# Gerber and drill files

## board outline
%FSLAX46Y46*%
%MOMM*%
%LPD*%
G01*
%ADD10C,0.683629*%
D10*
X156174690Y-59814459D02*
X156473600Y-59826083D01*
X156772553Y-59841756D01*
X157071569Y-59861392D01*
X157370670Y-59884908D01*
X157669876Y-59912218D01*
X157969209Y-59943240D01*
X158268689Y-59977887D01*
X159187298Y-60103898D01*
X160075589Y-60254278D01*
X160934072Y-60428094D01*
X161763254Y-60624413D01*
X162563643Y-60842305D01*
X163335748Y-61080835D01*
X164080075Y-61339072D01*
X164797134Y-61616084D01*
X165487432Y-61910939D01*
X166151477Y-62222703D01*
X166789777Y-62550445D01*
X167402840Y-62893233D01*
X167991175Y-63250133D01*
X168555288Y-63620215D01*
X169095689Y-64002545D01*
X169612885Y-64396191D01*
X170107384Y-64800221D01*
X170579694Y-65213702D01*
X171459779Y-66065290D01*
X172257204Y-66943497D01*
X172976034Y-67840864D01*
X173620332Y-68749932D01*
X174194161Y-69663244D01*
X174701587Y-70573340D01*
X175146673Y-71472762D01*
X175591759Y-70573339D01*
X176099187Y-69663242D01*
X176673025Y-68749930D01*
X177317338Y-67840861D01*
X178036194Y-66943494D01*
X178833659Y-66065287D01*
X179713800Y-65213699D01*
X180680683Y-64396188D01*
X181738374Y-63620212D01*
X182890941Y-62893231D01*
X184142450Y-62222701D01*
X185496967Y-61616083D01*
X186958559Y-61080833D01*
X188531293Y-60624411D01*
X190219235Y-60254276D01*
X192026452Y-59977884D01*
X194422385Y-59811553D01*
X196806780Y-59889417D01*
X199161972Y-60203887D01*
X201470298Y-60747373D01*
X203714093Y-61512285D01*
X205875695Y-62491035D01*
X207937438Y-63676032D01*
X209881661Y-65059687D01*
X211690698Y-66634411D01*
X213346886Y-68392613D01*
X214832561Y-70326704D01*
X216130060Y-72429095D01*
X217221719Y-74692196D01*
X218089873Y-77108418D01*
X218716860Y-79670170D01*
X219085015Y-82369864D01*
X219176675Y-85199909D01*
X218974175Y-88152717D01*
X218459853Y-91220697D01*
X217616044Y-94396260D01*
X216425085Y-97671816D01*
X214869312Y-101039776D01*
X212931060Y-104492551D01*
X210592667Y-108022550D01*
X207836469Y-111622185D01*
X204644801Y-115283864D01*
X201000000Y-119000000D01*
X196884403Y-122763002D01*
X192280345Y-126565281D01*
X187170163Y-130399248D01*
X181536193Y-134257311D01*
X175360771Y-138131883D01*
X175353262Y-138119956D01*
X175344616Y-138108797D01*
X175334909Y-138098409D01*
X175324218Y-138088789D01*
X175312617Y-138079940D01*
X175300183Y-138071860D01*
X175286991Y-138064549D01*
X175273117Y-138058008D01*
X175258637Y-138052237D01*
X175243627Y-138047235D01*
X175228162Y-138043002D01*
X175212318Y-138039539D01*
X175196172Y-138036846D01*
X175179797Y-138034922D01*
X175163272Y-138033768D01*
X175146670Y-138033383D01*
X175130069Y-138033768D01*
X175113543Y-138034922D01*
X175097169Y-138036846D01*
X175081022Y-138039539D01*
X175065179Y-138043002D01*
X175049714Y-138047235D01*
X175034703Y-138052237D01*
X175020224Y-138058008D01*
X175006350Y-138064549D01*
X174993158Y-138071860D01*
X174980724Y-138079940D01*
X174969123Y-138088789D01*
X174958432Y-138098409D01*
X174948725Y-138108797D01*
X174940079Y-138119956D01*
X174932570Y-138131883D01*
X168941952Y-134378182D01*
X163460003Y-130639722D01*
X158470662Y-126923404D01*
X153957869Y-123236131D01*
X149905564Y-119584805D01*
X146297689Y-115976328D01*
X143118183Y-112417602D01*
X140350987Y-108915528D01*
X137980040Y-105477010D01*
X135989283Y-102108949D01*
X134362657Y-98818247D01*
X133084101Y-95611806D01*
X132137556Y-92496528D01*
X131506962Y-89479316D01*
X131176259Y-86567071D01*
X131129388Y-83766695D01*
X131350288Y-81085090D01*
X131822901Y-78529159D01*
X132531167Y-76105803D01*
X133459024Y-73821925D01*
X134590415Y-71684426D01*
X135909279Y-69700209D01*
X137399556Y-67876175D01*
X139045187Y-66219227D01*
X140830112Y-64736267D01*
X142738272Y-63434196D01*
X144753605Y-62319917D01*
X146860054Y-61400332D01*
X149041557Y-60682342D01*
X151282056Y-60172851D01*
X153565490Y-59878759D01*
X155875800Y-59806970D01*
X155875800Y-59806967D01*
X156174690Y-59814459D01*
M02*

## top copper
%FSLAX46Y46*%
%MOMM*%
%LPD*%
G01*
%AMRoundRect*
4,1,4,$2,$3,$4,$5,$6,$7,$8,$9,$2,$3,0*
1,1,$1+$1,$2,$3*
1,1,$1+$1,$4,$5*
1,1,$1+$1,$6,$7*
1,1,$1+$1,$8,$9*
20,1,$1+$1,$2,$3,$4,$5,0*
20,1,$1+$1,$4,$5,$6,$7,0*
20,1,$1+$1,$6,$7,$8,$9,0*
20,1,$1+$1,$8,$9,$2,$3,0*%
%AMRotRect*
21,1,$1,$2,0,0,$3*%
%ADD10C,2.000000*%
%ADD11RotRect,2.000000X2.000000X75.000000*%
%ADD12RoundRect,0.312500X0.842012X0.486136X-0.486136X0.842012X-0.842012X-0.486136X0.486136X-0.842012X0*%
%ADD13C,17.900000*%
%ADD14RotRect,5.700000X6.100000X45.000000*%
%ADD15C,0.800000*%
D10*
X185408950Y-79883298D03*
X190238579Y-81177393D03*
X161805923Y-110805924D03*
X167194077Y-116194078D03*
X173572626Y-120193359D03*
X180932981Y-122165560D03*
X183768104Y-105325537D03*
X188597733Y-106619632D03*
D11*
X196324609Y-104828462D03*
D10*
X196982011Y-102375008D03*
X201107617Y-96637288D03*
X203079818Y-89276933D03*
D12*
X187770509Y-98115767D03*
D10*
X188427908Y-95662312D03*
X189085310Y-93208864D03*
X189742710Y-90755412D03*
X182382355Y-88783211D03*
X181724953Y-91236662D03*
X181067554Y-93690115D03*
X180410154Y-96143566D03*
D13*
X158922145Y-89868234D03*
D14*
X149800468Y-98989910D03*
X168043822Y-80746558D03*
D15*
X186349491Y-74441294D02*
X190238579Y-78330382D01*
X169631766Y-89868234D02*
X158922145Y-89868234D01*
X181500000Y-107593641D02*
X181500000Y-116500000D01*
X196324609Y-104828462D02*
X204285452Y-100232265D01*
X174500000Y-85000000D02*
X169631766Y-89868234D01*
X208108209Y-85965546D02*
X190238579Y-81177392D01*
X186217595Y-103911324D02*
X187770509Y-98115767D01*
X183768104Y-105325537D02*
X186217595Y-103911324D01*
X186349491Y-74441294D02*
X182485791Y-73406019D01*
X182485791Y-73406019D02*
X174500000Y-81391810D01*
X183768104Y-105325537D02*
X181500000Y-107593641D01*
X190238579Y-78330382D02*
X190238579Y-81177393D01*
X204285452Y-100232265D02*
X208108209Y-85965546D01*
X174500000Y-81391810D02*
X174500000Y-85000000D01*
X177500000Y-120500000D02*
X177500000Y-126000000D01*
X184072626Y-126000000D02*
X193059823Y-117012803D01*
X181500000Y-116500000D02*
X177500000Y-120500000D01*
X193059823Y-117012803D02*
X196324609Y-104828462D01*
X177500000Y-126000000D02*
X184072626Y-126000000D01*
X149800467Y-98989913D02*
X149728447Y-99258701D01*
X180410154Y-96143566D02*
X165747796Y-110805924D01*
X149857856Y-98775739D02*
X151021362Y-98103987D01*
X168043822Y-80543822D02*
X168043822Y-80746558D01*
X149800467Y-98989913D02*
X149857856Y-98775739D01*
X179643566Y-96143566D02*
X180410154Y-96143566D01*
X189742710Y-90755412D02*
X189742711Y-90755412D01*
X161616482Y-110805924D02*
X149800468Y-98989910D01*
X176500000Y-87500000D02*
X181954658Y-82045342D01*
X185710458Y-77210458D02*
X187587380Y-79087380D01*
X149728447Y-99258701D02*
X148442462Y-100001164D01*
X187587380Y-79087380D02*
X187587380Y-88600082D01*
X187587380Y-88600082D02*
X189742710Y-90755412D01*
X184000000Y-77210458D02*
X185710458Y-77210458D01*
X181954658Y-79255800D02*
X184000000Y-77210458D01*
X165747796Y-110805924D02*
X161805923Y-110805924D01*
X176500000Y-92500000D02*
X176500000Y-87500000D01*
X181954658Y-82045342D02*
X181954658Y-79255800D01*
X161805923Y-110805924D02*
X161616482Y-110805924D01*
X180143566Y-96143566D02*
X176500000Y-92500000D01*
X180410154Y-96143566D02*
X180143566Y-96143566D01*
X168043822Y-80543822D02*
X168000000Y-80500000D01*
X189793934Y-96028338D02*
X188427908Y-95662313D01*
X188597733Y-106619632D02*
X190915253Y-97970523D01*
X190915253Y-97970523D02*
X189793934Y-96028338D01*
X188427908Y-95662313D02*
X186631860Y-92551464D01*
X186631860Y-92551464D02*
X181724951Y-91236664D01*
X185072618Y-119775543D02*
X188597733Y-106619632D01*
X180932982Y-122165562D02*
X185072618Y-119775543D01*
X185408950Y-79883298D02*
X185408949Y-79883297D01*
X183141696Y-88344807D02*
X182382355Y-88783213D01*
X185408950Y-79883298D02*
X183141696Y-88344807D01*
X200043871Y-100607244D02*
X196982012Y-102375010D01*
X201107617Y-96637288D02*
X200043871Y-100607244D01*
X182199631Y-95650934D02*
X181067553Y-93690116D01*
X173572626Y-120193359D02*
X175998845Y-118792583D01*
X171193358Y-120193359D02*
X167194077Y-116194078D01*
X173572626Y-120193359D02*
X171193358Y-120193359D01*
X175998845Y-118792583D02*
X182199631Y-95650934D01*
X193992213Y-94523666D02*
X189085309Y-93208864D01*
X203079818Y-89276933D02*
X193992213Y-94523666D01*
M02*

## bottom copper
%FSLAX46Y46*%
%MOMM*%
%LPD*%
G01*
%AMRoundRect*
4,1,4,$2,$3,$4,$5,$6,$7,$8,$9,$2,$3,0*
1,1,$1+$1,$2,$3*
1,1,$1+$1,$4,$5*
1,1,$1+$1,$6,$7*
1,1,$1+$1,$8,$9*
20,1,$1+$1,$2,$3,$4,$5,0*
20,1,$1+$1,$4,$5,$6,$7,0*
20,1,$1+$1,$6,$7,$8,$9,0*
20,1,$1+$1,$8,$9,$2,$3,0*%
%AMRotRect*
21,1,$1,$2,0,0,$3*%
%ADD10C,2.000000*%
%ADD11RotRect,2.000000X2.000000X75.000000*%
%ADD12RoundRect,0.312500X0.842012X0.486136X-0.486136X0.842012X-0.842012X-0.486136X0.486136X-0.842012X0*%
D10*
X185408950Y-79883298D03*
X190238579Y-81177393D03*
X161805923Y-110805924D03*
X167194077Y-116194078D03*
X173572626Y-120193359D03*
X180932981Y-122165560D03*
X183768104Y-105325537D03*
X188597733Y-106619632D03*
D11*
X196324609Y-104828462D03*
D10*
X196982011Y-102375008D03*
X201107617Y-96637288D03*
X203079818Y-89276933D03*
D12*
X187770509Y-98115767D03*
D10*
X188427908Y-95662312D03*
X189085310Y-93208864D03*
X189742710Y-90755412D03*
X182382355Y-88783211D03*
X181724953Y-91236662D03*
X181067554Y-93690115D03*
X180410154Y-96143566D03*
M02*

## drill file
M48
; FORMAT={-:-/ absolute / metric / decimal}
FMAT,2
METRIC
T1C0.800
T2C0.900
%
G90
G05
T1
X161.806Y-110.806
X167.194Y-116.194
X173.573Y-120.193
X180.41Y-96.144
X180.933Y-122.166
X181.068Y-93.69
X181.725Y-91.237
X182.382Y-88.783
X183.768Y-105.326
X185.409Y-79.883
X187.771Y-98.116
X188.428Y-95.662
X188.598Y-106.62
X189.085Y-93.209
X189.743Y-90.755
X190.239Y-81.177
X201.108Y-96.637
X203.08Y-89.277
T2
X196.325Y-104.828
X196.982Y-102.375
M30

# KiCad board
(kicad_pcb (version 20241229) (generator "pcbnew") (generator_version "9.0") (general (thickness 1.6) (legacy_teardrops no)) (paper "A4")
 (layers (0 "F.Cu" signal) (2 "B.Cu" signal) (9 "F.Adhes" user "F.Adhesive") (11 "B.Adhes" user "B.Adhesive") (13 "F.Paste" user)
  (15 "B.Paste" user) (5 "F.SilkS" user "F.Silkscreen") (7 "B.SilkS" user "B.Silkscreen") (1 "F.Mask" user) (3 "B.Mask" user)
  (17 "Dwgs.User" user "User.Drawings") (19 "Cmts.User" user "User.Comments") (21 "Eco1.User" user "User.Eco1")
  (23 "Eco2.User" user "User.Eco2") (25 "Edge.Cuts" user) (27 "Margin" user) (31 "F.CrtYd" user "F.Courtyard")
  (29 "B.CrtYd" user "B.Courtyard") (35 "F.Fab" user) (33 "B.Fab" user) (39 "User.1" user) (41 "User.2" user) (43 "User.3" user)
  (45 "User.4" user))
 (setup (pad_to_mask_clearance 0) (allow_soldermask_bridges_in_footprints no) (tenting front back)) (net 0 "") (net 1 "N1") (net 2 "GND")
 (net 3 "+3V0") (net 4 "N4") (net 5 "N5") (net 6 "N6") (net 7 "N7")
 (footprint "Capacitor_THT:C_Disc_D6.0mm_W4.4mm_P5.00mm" (layer "F.Cu") (at 185.40895 79.883298 -15)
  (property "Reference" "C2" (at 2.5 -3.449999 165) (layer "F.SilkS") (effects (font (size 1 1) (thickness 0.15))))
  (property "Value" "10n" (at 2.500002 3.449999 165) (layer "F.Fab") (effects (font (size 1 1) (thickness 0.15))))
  (pad "1" thru_hole circle (at 0 0 345) (size 2 2) (drill 0.8) (layers "*.Cu" "*.Mask") (remove_unused_layers no) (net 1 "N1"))
  (pad "2" thru_hole circle (at 5 0 345) (size 2 2) (drill 0.8) (layers "*.Cu" "*.Mask") (remove_unused_layers no) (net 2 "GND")))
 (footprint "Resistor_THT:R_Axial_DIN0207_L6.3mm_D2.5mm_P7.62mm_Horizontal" (layer "F.Cu") (at 161.805923 110.805924 -45)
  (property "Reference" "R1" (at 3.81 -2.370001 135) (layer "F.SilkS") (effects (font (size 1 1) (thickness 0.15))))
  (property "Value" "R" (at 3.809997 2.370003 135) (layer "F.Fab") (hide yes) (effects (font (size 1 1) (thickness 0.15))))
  (pad "1" thru_hole circle (at 0 0 315) (size 2 2) (drill 0.8) (layers "*.Cu" "*.Mask") (remove_unused_layers no) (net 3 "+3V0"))
  (pad "2" thru_hole circle (at 7.62 0 315) (size 2 2) (drill 0.8) (layers "*.Cu" "*.Mask") (remove_unused_layers no) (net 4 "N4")))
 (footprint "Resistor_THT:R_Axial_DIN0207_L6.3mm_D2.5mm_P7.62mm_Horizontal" (layer "F.Cu") (at 173.572626 120.193359 -15)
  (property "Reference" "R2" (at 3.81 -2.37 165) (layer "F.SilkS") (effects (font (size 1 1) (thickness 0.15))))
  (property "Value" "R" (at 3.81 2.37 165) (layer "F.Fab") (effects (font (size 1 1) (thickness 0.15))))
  (pad "1" thru_hole circle (at 0 0 345) (size 2 2) (drill 0.8) (layers "*.Cu" "*.Mask") (remove_unused_layers no) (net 4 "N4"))
  (pad "2" thru_hole circle (at 7.62 0 345) (size 2 2) (drill 0.8) (layers "*.Cu" "*.Mask") (remove_unused_layers no) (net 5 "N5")))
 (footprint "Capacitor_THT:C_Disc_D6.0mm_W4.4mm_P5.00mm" (layer "F.Cu") (at 183.768104 105.325537 -15)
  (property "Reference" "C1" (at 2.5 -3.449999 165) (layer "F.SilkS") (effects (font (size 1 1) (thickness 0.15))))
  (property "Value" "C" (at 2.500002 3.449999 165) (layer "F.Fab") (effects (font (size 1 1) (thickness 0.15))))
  (pad "1" thru_hole circle (at 0 0 345) (size 2 2) (drill 0.8) (layers "*.Cu" "*.Mask") (remove_unused_layers no) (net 2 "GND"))
  (pad "2" thru_hole circle (at 5 0 345) (size 2 2) (drill 0.8) (layers "*.Cu" "*.Mask") (remove_unused_layers no) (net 5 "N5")))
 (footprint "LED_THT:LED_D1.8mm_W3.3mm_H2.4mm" (layer "F.Cu") (at 196.324609 104.828462 75)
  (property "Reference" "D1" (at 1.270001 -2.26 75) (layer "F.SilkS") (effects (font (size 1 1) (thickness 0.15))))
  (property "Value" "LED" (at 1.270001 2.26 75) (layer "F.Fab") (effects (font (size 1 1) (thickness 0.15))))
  (pad "1" thru_hole rect (at 0 0 75) (size 2 2) (drill 0.9) (layers "*.Cu" "*.Mask") (remove_unused_layers no) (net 2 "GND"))
  (pad "2" thru_hole circle (at 2.540003 0.000001 75) (size 2 2) (drill 0.9) (layers "*.Cu" "*.Mask") (remove_unused_layers no) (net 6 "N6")))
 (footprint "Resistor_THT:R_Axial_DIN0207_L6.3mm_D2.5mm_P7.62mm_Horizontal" (layer "F.Cu") (at 201.107617 96.637288 75)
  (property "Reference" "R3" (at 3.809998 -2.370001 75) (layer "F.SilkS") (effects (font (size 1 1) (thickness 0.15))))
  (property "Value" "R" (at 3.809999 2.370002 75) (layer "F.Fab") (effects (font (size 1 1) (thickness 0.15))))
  (pad "1" thru_hole circle (at 0 0 75) (size 2 2) (drill 0.8) (layers "*.Cu" "*.Mask") (remove_unused_layers no) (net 6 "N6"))
  (pad "2" thru_hole circle (at 7.62 0 75) (size 2 2) (drill 0.8) (layers "*.Cu" "*.Mask") (remove_unused_layers no) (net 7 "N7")))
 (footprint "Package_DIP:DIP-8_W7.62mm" (layer "F.Cu") (at 187.770509 98.115767 165)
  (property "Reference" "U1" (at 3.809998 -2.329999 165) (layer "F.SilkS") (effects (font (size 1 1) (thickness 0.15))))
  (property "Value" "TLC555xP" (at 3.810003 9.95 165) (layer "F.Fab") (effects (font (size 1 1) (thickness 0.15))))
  (pad "1" thru_hole roundrect (at 0 0 165) (size 2 2) (drill 0.8) (layers "*.Cu" "*.Mask") (remove_unused_layers no)
   (roundrect_rratio 0.15625) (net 2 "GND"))
  (pad "2" thru_hole circle (at 0.000002 2.540003 165) (size 2 2) (drill 0.8) (layers "*.Cu" "*.Mask") (remove_unused_layers no)
   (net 5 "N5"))
  (pad "3" thru_hole circle (at 0 5.08 165) (size 2 2) (drill 0.8) (layers "*.Cu" "*.Mask") (remove_unused_layers no) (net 7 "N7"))
  (pad "4" thru_hole circle (at 0 7.62 165) (size 2 2) (drill 0.8) (layers "*.Cu" "*.Mask") (remove_unused_layers no) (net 3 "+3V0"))
  (pad "5" thru_hole circle (at 7.62 7.62 165) (size 2 2) (drill 0.8) (layers "*.Cu" "*.Mask") (remove_unused_layers no) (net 1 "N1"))
  (pad "6" thru_hole circle (at 7.620002 5.08 165) (size 2 2) (drill 0.8) (layers "*.Cu" "*.Mask") (remove_unused_layers no) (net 5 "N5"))
  (pad "7" thru_hole circle (at 7.62 2.539999 165) (size 2 2) (drill 0.8) (layers "*.Cu" "*.Mask") (remove_unused_layers no) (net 4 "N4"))
  (pad "8" thru_hole circle (at 7.62 0 165) (size 2 2) (drill 0.8) (layers "*.Cu" "*.Mask") (remove_unused_layers no) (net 3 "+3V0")))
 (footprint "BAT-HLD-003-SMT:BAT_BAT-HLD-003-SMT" (layer "F.Cu") (at 158.922145 89.868234 45)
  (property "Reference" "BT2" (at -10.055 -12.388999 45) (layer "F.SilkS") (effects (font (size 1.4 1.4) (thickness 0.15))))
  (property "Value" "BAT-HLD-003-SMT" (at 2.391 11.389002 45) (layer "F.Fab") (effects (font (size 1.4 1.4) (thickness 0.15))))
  (pad "N" smd circle (at 0 0 45) (size 17.9 17.9) (layers "F.Cu" "F.Mask") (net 2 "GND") (solder_mask_margin 0.102))
  (pad "P1" smd rect (at -12.899999 -0.000001 45) (size 5.7 6.1) (layers "F.Cu" "F.Mask" "F.Paste") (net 3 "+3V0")
   (solder_mask_margin 0.102))
  (pad "P2" smd rect (at 12.899999 0.000001 45) (size 5.7 6.1) (layers "F.Cu" "F.Mask" "F.Paste") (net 3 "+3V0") (solder_mask_margin 0.102)))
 (gr_poly
  (pts (xy 156.17469 59.814459) (xy 156.4736 59.826083) (xy 156.772553 59.841756) (xy 157.071569 59.861392) (xy 157.37067 59.884908)
   (xy 157.669876 59.912218) (xy 157.969209 59.94324) (xy 158.268689 59.977887) (xy 159.187298 60.103898) (xy 160.075589 60.254278)
   (xy 160.934072 60.428094) (xy 161.763254 60.624413) (xy 162.563643 60.842305) (xy 163.335748 61.080835) (xy 164.080075 61.339072)
   (xy 164.797134 61.616084) (xy 165.487432 61.910939) (xy 166.151477 62.222703) (xy 166.789777 62.550445) (xy 167.40284 62.893233)
   (xy 167.991175 63.250133) (xy 168.555288 63.620215) (xy 169.095689 64.002545) (xy 169.612885 64.396191) (xy 170.107384 64.800221)
   (xy 170.579694 65.213702) (xy 171.459779 66.06529) (xy 172.257204 66.943497) (xy 172.976034 67.840864) (xy 173.620332 68.749932)
   (xy 174.194161 69.663244) (xy 174.701587 70.57334) (xy 175.146673 71.472762) (xy 175.591759 70.573339) (xy 176.099187 69.663242)
   (xy 176.673025 68.74993) (xy 177.317338 67.840861) (xy 178.036194 66.943494) (xy 178.833659 66.065287) (xy 179.7138 65.213699)
   (xy 180.680683 64.396188) (xy 181.738374 63.620212) (xy 182.890941 62.893231) (xy 184.14245 62.222701) (xy 185.496967 61.616083)
   (xy 186.958559 61.080833) (xy 188.531293 60.624411) (xy 190.219235 60.254276) (xy 192.026452 59.977884) (xy 194.422385 59.811553)
   (xy 196.80678 59.889417) (xy 199.161972 60.203887) (xy 201.470298 60.747373) (xy 203.714093 61.512285) (xy 205.875695 62.491035)
   (xy 207.937438 63.676032) (xy 209.881661 65.059687) (xy 211.690698 66.634411) (xy 213.346886 68.392613) (xy 214.832561 70.326704)
   (xy 216.13006 72.429095) (xy 217.221719 74.692196) (xy 218.089873 77.108418) (xy 218.71686 79.67017) (xy 219.085015 82.369864)
   (xy 219.176675 85.199909) (xy 218.974175 88.152717) (xy 218.459853 91.220697) (xy 217.616044 94.39626) (xy 216.425085 97.671816)
   (xy 214.869312 101.039776) (xy 212.93106 104.492551) (xy 210.592667 108.02255) (xy 207.836469 111.622185) (xy 204.644801 115.283864)
   (xy 201 119) (xy 196.884403 122.763002) (xy 192.280345 126.565281) (xy 187.170163 130.399248) (xy 181.536193 134.257311)
   (xy 175.360771 138.131883) (xy 175.353262 138.119956) (xy 175.344616 138.108797) (xy 175.334909 138.098409) (xy 175.324218 138.088789)
   (xy 175.312617 138.07994) (xy 175.300183 138.07186) (xy 175.286991 138.064549) (xy 175.273117 138.058008) (xy 175.258637 138.052237)
   (xy 175.243627 138.047235) (xy 175.228162 138.043002) (xy 175.212318 138.039539) (xy 175.196172 138.036846) (xy 175.179797 138.034922)
   (xy 175.163272 138.033768) (xy 175.14667 138.033383) (xy 175.130069 138.033768) (xy 175.113543 138.034922) (xy 175.097169 138.036846)
   (xy 175.081022 138.039539) (xy 175.065179 138.043002) (xy 175.049714 138.047235) (xy 175.034703 138.052237) (xy 175.020224 138.058008)
   (xy 175.00635 138.064549) (xy 174.993158 138.07186) (xy 174.980724 138.07994) (xy 174.969123 138.088789) (xy 174.958432 138.098409)
   (xy 174.948725 138.108797) (xy 174.940079 138.119956) (xy 174.93257 138.131883) (xy 168.941952 134.378182) (xy 163.460003 130.639722)
   (xy 158.470662 126.923404) (xy 153.957869 123.236131) (xy 149.905564 119.584805) (xy 146.297689 115.976328) (xy 143.118183 112.417602)
   (xy 140.350987 108.915528) (xy 137.98004 105.47701) (xy 135.989283 102.108949) (xy 134.362657 98.818247) (xy 133.084101 95.611806)
   (xy 132.137556 92.496528) (xy 131.506962 89.479316) (xy 131.176259 86.567071) (xy 131.129388 83.766695) (xy 131.350288 81.08509)
   (xy 131.822901 78.529159) (xy 132.531167 76.105803) (xy 133.459024 73.821925) (xy 134.590415 71.684426) (xy 135.909279 69.700209)
   (xy 137.399556 67.876175) (xy 139.045187 66.219227) (xy 140.830112 64.736267) (xy 142.738272 63.434196) (xy 144.753605 62.319917)
   (xy 146.860054 61.400332) (xy 149.041557 60.682342) (xy 151.282056 60.172851) (xy 153.56549 59.878759) (xy 155.8758 59.80697)
   (xy 155.8758 59.806967))
  (stroke (width 0.683629) (type solid)) (fill no) (layer "Edge.Cuts"))
 (segment (start 186.349491 74.441294) (end 190.238579 78.330382) (width 0.8) (layer "F.Cu") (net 2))
 (segment (start 169.631766 89.868234) (end 158.922145 89.868234) (width 0.8) (layer "F.Cu") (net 2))
 (segment (start 181.5 107.593641) (end 181.5 116.5) (width 0.8) (layer "F.Cu") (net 2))
 (segment (start 196.324609 104.828462) (end 204.285452 100.232265) (width 0.8) (layer "F.Cu") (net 2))
 (segment (start 174.5 85) (end 169.631766 89.868234) (width 0.8) (layer "F.Cu") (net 2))
 (segment (start 208.108209 85.965546) (end 190.238579 81.177392) (width 0.8) (layer "F.Cu") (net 2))
 (segment (start 186.217595 103.911324) (end 187.770509 98.115767) (width 0.8) (layer "F.Cu") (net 2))
 (segment (start 183.768104 105.325537) (end 186.217595 103.911324) (width 0.8) (layer "F.Cu") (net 2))
 (segment (start 186.349491 74.441294) (end 182.485791 73.406019) (width 0.8) (layer "F.Cu") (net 2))
 (segment (start 182.485791 73.406019) (end 174.5 81.39181) (width 0.8) (layer "F.Cu") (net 2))
 (segment (start 183.768104 105.325537) (end 181.5 107.593641) (width 0.8) (layer "F.Cu") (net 2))
 (segment (start 190.238579 78.330382) (end 190.238579 81.177393) (width 0.8) (layer "F.Cu") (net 2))
 (segment (start 204.285452 100.232265) (end 208.108209 85.965546) (width 0.8) (layer "F.Cu") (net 2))
 (segment (start 174.5 81.39181) (end 174.5 85) (width 0.8) (layer "F.Cu") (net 2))
 (segment (start 177.5 120.5) (end 177.5 126) (width 0.8) (layer "F.Cu") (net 2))
 (segment (start 184.072626 126) (end 193.059823 117.012803) (width 0.8) (layer "F.Cu") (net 2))
 (segment (start 181.5 116.5) (end 177.5 120.5) (width 0.8) (layer "F.Cu") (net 2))
 (segment (start 193.059823 117.012803) (end 196.324609 104.828462) (width 0.8) (layer "F.Cu") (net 2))
 (segment (start 177.5 126) (end 184.072626 126) (width 0.8) (layer "F.Cu") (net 2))
 (segment (start 149.800467 98.989913) (end 149.728447 99.258701) (width 0.8) (layer "F.Cu") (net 3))
 (segment (start 180.410154 96.143566) (end 165.747796 110.805924) (width 0.8) (layer "F.Cu") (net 3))
 (segment (start 149.857856 98.775739) (end 151.021362 98.103987) (width 0.8) (layer "F.Cu") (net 3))
 (segment (start 168.043822 80.543822) (end 168.043822 80.746558) (width 0.8) (layer "F.Cu") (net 3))
 (segment (start 149.800467 98.989913) (end 149.857856 98.775739) (width 0.8) (layer "F.Cu") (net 3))
 (segment (start 179.643566 96.143566) (end 180.410154 96.143566) (width 0.8) (layer "F.Cu") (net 3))
 (segment (start 189.74271 90.755412) (end 189.742711 90.755412) (width 0.8) (layer "F.Cu") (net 3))
 (segment (start 161.616482 110.805924) (end 149.800468 98.98991) (width 0.8) (layer "F.Cu") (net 3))
 (segment (start 176.5 87.5) (end 181.954658 82.045342) (width 0.8) (layer "F.Cu") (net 3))
 (segment (start 185.710458 77.210458) (end 187.58738 79.08738) (width 0.8) (layer "F.Cu") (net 3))
 (segment (start 149.728447 99.258701) (end 148.442462 100.001164) (width 0.8) (layer "F.Cu") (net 3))
 (segment (start 187.58738 79.08738) (end 187.58738 88.600082) (width 0.8) (layer "F.Cu") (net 3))
 (segment (start 187.58738 88.600082) (end 189.74271 90.755412) (width 0.8) (layer "F.Cu") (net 3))
 (segment (start 184 77.210458) (end 185.710458 77.210458) (width 0.8) (layer "F.Cu") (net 3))
 (segment (start 181.954658 79.2558) (end 184 77.210458) (width 0.8) (layer "F.Cu") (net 3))
 (segment (start 165.747796 110.805924) (end 161.805923 110.805924) (width 0.8) (layer "F.Cu") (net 3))
 (segment (start 176.5 92.5) (end 176.5 87.5) (width 0.8) (layer "F.Cu") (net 3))
 (segment (start 181.954658 82.045342) (end 181.954658 79.2558) (width 0.8) (layer "F.Cu") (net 3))
 (segment (start 161.805923 110.805924) (end 161.616482 110.805924) (width 0.8) (layer "F.Cu") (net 3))
 (segment (start 180.143566 96.143566) (end 176.5 92.5) (width 0.8) (layer "F.Cu") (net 3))
 (segment (start 180.410154 96.143566) (end 180.143566 96.143566) (width 0.8) (layer "F.Cu") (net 3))
 (segment (start 168.043822 80.543822) (end 168 80.5) (width 0.8) (layer "F.Cu") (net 3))
 (segment (start 189.793934 96.028338) (end 188.427908 95.662313) (width 0.8) (layer "F.Cu") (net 5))
 (segment (start 188.597733 106.619632) (end 190.915253 97.970523) (width 0.8) (layer "F.Cu") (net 5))
 (segment (start 190.915253 97.970523) (end 189.793934 96.028338) (width 0.8) (layer "F.Cu") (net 5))
 (segment (start 188.427908 95.662313) (end 186.63186 92.551464) (width 0.8) (layer "F.Cu") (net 5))
 (segment (start 186.63186 92.551464) (end 181.724951 91.236664) (width 0.8) (layer "F.Cu") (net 5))
 (segment (start 185.072618 119.775543) (end 188.597733 106.619632) (width 0.8) (layer "F.Cu") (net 5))
 (segment (start 180.932982 122.165562) (end 185.072618 119.775543) (width 0.8) (layer "F.Cu") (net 5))
 (segment (start 185.40895 79.883298) (end 185.408949 79.883297) (width 0.8) (layer "F.Cu") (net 1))
 (segment (start 183.141696 88.344807) (end 182.382355 88.783213) (width 0.8) (layer "F.Cu") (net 1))
 (segment (start 185.40895 79.883298) (end 183.141696 88.344807) (width 0.8) (layer "F.Cu") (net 1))
 (segment (start 200.043871 100.607244) (end 196.982012 102.37501) (width 0.8) (layer "F.Cu") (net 6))
 (segment (start 201.107617 96.637288) (end 200.043871 100.607244) (width 0.8) (layer "F.Cu") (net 6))
 (segment (start 182.199631 95.650934) (end 181.067553 93.690116) (width 0.8) (layer "F.Cu") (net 4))
 (segment (start 173.572626 120.193359) (end 175.998845 118.792583) (width 0.8) (layer "F.Cu") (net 4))
 (segment (start 171.193358 120.193359) (end 167.194077 116.194078) (width 0.8) (layer "F.Cu") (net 4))
 (segment (start 173.572626 120.193359) (end 171.193358 120.193359) (width 0.8) (layer "F.Cu") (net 4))
 (segment (start 175.998845 118.792583) (end 182.199631 95.650934) (width 0.8) (layer "F.Cu") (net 4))
 (segment (start 193.992213 94.523666) (end 189.085309 93.208864) (width 0.8) (layer "F.Cu") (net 7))
 (segment (start 203.079818 89.276933) (end 193.992213 94.523666) (width 0.8) (layer "F.Cu") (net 7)))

